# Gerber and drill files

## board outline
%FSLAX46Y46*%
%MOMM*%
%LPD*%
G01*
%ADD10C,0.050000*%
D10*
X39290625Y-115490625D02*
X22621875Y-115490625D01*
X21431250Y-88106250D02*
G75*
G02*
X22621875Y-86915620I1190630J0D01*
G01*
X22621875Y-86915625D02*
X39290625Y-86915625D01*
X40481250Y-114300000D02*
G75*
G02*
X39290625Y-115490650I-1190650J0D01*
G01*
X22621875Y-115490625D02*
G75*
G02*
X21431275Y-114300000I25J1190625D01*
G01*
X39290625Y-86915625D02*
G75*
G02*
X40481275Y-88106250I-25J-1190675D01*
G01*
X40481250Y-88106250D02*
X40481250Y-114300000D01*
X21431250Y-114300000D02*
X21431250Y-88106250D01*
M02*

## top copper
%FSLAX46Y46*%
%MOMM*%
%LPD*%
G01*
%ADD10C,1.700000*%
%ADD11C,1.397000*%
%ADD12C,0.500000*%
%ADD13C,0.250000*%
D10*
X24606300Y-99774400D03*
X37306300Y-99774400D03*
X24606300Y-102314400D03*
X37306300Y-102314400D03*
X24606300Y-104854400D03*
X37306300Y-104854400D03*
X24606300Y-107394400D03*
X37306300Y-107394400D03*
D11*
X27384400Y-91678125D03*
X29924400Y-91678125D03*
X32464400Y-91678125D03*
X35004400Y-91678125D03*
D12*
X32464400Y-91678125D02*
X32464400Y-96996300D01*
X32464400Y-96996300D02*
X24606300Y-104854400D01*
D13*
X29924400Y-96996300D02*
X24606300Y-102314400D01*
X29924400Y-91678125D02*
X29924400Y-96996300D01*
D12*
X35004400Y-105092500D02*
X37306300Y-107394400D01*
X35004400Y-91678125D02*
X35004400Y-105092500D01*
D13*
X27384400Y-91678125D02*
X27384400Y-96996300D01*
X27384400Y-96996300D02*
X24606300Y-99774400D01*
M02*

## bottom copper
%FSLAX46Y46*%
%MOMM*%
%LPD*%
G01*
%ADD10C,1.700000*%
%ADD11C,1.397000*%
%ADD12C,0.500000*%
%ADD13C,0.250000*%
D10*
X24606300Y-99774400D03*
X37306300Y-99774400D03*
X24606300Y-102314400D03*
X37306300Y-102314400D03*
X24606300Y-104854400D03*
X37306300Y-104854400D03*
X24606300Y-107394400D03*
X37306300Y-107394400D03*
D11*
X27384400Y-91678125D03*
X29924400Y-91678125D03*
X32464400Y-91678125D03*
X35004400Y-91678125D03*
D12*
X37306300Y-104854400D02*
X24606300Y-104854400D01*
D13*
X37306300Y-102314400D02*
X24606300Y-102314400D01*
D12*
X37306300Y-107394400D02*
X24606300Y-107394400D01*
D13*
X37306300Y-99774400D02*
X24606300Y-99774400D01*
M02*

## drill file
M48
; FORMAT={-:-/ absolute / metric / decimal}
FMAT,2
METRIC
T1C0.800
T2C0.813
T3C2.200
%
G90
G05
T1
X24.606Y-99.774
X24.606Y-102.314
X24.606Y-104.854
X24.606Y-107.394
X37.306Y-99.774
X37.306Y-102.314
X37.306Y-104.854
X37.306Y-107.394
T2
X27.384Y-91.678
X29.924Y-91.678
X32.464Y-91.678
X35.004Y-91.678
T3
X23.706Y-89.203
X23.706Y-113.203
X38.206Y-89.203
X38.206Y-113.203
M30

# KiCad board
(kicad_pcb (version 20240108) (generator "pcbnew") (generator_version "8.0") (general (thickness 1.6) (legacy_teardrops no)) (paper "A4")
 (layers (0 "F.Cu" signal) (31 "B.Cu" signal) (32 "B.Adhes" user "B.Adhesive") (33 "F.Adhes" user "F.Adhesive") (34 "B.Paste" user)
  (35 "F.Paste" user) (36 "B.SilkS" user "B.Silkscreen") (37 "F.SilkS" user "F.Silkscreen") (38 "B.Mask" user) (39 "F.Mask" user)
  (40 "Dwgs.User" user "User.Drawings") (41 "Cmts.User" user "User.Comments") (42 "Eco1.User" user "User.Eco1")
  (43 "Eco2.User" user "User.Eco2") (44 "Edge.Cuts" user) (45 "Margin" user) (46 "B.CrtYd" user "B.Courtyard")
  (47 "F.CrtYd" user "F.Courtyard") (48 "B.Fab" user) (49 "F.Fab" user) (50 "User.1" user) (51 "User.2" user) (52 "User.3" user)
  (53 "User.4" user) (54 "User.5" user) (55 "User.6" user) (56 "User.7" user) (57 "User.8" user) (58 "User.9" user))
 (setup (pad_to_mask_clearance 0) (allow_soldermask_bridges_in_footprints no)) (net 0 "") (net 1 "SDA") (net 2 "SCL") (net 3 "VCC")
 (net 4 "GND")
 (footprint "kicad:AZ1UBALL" (layer "F.Cu") (at 30.9563 103.5844)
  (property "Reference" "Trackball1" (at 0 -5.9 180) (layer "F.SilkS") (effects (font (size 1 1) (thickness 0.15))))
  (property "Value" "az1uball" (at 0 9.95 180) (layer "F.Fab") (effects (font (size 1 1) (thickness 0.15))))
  (pad "1" thru_hole circle (at -6.35 -3.81) (size 1.7 1.7) (drill 0.8) (layers "*.Cu" "*.Mask") (remove_unused_layers no) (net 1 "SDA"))
  (pad "1" thru_hole circle (at 6.35 -3.81) (size 1.7 1.7) (drill 0.8) (layers "*.Cu" "*.Mask") (remove_unused_layers no) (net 1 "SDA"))
  (pad "2" thru_hole circle (at -6.35 -1.27) (size 1.7 1.7) (drill 0.8) (layers "*.Cu" "*.Mask") (remove_unused_layers no) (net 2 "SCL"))
  (pad "2" thru_hole circle (at 6.35 -1.27) (size 1.7 1.7) (drill 0.8) (layers "*.Cu" "*.Mask") (remove_unused_layers no) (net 2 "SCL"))
  (pad "3" thru_hole circle (at -6.35 1.27) (size 1.7 1.7) (drill 0.8) (layers "*.Cu" "*.Mask") (remove_unused_layers no) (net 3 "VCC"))
  (pad "3" thru_hole circle (at 6.35 1.27) (size 1.7 1.7) (drill 0.8) (layers "*.Cu" "*.Mask") (remove_unused_layers no) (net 3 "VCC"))
  (pad "4" thru_hole circle (at -6.35 3.81) (size 1.7 1.7) (drill 0.8) (layers "*.Cu" "*.Mask") (remove_unused_layers no) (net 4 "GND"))
  (pad "4" thru_hole circle (at 6.35 3.81) (size 1.7 1.7) (drill 0.8) (layers "*.Cu" "*.Mask") (remove_unused_layers no) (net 4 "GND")))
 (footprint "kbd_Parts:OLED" (layer "F.Cu") (at 27.3844 91.678125)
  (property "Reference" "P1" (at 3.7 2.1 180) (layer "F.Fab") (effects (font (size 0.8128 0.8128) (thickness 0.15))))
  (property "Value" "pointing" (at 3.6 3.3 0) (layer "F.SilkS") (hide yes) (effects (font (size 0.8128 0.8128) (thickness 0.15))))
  (pad "1" thru_hole circle (at 0 0) (size 1.397 1.397) (drill 0.8128) (layers "*.Cu" "*.Mask" "F.SilkS") (remove_unused_layers no)
   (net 1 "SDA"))
  (pad "2" thru_hole circle (at 2.54 0) (size 1.397 1.397) (drill 0.8128) (layers "*.Cu" "*.Mask" "F.SilkS") (remove_unused_layers no)
   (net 2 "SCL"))
  (pad "3" thru_hole circle (at 5.08 0) (size 1.397 1.397) (drill 0.8128) (layers "*.Cu" "*.Mask" "F.SilkS") (remove_unused_layers no)
   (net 3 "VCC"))
  (pad "4" thru_hole circle (at 7.62 0) (size 1.397 1.397) (drill 0.8128) (layers "*.Cu" "*.Mask" "F.SilkS") (remove_unused_layers no)
   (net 4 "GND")))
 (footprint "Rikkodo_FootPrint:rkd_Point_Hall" (layer "F.Cu") (at 30.9563 101.2031)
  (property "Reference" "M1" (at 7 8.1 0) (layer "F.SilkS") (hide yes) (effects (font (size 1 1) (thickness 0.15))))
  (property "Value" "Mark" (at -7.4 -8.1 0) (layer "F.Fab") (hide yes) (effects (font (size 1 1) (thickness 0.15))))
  (pad "" np_thru_hole circle (at -7.25 -12) (size 2.2 2.2) (drill 2.2) (layers "*.Cu" "*.Mask"))
  (pad "" np_thru_hole circle (at -7.25 12) (size 2.2 2.2) (drill 2.2) (layers "*.Cu" "*.Mask"))
  (pad "" np_thru_hole circle (at 7.25 -12) (size 2.2 2.2) (drill 2.2) (layers "*.Cu" "*.Mask"))
  (pad "" np_thru_hole circle (at 7.25 12) (size 2.2 2.2) (drill 2.2) (layers "*.Cu" "*.Mask")))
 (gr_line (start 39.290625 115.490625) (end 22.621875 115.490625) (stroke (width 0.05) (type default)) (layer "Edge.Cuts"))
 (gr_arc (start 21.43125 88.10625) (mid 21.779976 87.264351) (end 22.621875 86.915625) (stroke (width 0.05) (type default))
  (layer "Edge.Cuts"))
 (gr_line (start 22.621875 86.915625) (end 39.290625 86.915625) (stroke (width 0.05) (type default)) (layer "Edge.Cuts"))
 (gr_arc (start 40.48125 114.3) (mid 40.132524 115.141899) (end 39.290625 115.490625) (stroke (width 0.05) (type default))
  (layer "Edge.Cuts"))
 (gr_arc (start 22.621875 115.490625) (mid 21.779976 115.141899) (end 21.43125 114.3) (stroke (width 0.05) (type default))
  (layer "Edge.Cuts"))
 (gr_arc (start 39.290625 86.915625) (mid 40.132524 87.264351) (end 40.48125 88.10625) (stroke (width 0.05) (type default))
  (layer "Edge.Cuts"))
 (gr_line (start 40.48125 88.10625) (end 40.48125 114.3) (stroke (width 0.05) (type default)) (layer "Edge.Cuts"))
 (gr_line (start 21.43125 114.3) (end 21.43125 88.10625) (stroke (width 0.05) (type default)) (layer "Edge.Cuts"))
 (segment (start 32.4644 91.678125) (end 32.4644 96.9963) (width 0.5) (layer "F.Cu") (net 3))
 (segment (start 32.4644 96.9963) (end 24.6063 104.8544) (width 0.5) (layer "F.Cu") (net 3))
 (segment (start 37.3063 104.8544) (end 24.6063 104.8544) (width 0.5) (layer "B.Cu") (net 3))
 (segment (start 29.9244 96.9963) (end 24.6063 102.3144) (width 0.25) (layer "F.Cu") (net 2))
 (segment (start 29.9244 91.678125) (end 29.9244 96.9963) (width 0.25) (layer "F.Cu") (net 2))
 (segment (start 37.3063 102.3144) (end 24.6063 102.3144) (width 0.25) (layer "B.Cu") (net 2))
 (segment (start 35.0044 105.0925) (end 37.3063 107.3944) (width 0.5) (layer "F.Cu") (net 4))
 (segment (start 35.0044 91.678125) (end 35.0044 105.0925) (width 0.5) (layer "F.Cu") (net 4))
 (segment (start 37.3063 107.3944) (end 24.6063 107.3944) (width 0.5) (layer "B.Cu") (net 4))
 (segment (start 27.3844 91.678125) (end 27.3844 96.9963) (width 0.25) (layer "F.Cu") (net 1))
 (segment (start 27.3844 96.9963) (end 24.6063 99.7744) (width 0.25) (layer "F.Cu") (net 1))
 (segment (start 37.3063 99.7744) (end 24.6063 99.7744) (width 0.25) (layer "B.Cu") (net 1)))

